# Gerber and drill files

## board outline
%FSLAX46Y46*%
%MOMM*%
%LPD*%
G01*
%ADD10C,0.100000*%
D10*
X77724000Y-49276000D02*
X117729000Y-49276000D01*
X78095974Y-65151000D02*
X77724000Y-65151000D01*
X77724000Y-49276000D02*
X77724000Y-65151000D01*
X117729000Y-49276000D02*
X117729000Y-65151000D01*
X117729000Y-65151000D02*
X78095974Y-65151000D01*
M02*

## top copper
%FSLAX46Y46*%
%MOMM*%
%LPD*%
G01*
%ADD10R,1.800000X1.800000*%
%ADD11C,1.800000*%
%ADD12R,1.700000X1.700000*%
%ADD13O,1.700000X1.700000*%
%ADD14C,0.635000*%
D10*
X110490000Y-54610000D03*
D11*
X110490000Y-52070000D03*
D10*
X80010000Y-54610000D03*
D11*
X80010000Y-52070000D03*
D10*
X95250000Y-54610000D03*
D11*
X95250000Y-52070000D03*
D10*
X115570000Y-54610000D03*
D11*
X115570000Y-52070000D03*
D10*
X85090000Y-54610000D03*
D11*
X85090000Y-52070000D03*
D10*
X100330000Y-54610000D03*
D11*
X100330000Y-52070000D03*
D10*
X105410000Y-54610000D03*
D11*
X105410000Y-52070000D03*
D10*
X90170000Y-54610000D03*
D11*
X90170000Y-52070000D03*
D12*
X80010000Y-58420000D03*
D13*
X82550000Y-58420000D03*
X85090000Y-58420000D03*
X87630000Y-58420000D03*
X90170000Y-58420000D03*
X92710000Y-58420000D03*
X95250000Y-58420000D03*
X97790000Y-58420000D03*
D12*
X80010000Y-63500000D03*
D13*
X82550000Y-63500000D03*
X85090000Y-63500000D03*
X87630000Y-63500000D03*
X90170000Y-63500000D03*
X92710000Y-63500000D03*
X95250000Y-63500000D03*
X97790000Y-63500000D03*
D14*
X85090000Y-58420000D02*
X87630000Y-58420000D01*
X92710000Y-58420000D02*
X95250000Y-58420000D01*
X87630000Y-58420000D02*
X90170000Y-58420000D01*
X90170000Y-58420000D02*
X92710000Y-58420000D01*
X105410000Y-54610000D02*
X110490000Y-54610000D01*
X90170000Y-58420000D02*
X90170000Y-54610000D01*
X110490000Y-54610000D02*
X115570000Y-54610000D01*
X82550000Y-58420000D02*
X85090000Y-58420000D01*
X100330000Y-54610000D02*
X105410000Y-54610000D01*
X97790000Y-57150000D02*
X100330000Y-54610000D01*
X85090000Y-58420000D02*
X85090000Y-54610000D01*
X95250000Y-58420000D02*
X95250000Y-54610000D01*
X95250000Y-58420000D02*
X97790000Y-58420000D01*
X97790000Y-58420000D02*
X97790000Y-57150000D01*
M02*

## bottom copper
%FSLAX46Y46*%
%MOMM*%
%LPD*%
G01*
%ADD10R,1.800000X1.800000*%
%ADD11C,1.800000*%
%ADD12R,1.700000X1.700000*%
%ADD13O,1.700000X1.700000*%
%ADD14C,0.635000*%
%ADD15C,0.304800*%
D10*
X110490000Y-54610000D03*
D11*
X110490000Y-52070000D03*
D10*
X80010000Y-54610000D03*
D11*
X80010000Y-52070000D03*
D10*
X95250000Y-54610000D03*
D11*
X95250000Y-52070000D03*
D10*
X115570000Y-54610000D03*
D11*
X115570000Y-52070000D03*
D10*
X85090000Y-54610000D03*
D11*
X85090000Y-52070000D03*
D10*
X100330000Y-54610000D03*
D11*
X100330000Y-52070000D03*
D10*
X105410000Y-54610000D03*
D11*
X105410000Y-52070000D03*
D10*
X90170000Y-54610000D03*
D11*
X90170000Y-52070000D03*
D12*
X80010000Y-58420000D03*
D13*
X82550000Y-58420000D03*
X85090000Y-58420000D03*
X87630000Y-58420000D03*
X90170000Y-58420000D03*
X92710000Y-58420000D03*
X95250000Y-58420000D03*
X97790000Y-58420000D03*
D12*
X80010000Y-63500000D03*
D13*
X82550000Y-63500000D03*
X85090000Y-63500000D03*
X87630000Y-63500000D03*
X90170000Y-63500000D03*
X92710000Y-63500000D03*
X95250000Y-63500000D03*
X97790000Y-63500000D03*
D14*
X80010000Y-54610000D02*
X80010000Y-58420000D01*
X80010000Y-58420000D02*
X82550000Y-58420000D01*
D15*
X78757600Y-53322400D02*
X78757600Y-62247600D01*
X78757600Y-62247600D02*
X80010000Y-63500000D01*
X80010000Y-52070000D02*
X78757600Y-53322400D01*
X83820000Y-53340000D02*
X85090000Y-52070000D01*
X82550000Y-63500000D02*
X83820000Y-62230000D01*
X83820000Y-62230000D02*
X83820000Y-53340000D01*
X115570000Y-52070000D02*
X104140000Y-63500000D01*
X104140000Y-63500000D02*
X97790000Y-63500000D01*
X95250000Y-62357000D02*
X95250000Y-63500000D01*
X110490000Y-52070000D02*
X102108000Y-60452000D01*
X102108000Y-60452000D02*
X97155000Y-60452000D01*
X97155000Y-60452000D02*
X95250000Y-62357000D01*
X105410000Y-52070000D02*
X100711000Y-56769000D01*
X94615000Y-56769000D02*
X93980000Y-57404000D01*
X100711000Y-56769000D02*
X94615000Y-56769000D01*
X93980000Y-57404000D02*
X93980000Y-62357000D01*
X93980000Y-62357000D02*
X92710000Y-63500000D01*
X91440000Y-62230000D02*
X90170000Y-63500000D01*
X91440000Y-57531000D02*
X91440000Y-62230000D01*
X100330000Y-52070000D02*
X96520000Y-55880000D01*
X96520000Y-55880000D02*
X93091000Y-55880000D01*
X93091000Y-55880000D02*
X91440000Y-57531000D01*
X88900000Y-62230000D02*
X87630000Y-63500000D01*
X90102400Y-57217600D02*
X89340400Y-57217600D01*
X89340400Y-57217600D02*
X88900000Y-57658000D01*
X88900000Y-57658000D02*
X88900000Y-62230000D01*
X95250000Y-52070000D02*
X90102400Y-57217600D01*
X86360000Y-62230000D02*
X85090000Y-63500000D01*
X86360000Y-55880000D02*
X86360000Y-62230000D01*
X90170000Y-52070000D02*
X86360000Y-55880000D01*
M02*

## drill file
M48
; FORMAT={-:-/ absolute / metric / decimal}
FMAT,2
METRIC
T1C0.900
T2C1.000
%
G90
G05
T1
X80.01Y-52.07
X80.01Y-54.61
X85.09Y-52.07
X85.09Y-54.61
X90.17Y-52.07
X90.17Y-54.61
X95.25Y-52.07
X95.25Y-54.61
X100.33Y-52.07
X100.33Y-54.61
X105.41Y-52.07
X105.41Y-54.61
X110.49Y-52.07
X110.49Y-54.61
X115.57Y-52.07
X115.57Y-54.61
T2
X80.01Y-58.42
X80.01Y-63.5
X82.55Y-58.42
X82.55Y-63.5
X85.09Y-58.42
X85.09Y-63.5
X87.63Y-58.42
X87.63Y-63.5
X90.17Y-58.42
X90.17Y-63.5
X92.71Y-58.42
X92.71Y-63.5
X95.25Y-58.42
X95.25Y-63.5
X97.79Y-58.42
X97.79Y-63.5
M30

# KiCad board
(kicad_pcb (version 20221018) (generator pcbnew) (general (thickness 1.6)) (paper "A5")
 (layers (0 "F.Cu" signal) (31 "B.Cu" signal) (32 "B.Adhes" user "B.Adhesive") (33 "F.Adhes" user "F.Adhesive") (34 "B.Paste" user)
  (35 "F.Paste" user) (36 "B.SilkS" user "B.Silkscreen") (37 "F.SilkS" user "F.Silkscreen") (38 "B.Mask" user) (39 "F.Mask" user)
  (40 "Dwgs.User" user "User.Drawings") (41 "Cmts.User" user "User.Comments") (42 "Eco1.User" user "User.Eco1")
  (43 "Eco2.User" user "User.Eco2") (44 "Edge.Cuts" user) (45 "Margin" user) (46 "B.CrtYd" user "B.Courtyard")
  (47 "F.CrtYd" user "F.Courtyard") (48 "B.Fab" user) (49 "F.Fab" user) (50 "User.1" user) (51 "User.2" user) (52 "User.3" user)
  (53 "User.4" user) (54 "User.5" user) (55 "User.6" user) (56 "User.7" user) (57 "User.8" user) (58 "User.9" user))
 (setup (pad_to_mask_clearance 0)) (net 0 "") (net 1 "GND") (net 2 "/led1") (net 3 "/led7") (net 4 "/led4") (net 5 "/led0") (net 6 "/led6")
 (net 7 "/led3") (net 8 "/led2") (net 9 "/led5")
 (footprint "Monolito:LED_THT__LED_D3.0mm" (layer "F.Cu") (at 110.49 54.61 90)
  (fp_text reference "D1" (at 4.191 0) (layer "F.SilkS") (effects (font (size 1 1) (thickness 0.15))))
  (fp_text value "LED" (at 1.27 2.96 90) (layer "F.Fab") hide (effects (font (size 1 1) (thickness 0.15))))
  (pad "1" thru_hole rect (at 0 0 90) (size 1.8 1.8) (drill 0.9) (layers "*.Cu" "*.Mask") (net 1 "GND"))
  (pad "2" thru_hole circle (at 2.54 0 90) (size 1.8 1.8) (drill 0.9) (layers "*.Cu" "*.Mask") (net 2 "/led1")))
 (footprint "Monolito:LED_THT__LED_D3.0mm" (layer "F.Cu") (at 80.01 54.61 90)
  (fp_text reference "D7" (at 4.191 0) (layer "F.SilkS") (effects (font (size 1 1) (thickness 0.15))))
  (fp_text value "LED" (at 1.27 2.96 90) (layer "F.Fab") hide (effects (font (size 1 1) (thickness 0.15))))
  (pad "1" thru_hole rect (at 0 0 90) (size 1.8 1.8) (drill 0.9) (layers "*.Cu" "*.Mask") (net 1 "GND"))
  (pad "2" thru_hole circle (at 2.54 0 90) (size 1.8 1.8) (drill 0.9) (layers "*.Cu" "*.Mask") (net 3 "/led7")))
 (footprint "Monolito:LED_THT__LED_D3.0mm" (layer "F.Cu") (at 95.25 54.61 90)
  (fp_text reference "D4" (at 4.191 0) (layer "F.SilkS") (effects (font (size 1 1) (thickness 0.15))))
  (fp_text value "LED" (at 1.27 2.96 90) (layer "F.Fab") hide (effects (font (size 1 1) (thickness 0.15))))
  (pad "1" thru_hole rect (at 0 0 90) (size 1.8 1.8) (drill 0.9) (layers "*.Cu" "*.Mask") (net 1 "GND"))
  (pad "2" thru_hole circle (at 2.54 0 90) (size 1.8 1.8) (drill 0.9) (layers "*.Cu" "*.Mask") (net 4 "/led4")))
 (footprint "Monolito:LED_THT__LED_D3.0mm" (layer "F.Cu") (at 115.57 54.61 90)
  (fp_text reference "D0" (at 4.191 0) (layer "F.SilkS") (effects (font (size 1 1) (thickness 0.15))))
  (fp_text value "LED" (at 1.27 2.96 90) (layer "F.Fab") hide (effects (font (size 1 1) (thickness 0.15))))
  (pad "1" thru_hole rect (at 0 0 90) (size 1.8 1.8) (drill 0.9) (layers "*.Cu" "*.Mask") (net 1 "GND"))
  (pad "2" thru_hole circle (at 2.54 0 90) (size 1.8 1.8) (drill 0.9) (layers "*.Cu" "*.Mask") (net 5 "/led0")))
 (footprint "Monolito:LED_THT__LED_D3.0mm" (layer "F.Cu") (at 85.09 54.61 90)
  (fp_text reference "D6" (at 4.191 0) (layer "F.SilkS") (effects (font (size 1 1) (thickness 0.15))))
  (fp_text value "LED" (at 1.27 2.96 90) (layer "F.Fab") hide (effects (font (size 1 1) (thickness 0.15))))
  (pad "1" thru_hole rect (at 0 0 90) (size 1.8 1.8) (drill 0.9) (layers "*.Cu" "*.Mask") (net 1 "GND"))
  (pad "2" thru_hole circle (at 2.54 0 90) (size 1.8 1.8) (drill 0.9) (layers "*.Cu" "*.Mask") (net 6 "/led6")))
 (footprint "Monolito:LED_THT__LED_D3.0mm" (layer "F.Cu") (at 100.33 54.61 90)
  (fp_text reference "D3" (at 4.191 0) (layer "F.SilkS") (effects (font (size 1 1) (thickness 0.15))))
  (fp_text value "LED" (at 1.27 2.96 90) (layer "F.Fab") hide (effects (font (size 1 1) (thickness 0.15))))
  (pad "1" thru_hole rect (at 0 0 90) (size 1.8 1.8) (drill 0.9) (layers "*.Cu" "*.Mask") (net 1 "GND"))
  (pad "2" thru_hole circle (at 2.54 0 90) (size 1.8 1.8) (drill 0.9) (layers "*.Cu" "*.Mask") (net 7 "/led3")))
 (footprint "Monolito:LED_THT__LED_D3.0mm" (layer "F.Cu") (at 105.41 54.61 90)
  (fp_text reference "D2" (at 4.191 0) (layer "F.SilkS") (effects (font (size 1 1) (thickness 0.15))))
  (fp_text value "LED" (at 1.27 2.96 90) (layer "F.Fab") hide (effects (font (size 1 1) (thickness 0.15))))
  (pad "1" thru_hole rect (at 0 0 90) (size 1.8 1.8) (drill 0.9) (layers "*.Cu" "*.Mask") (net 1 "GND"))
  (pad "2" thru_hole circle (at 2.54 0 90) (size 1.8 1.8) (drill 0.9) (layers "*.Cu" "*.Mask") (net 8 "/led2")))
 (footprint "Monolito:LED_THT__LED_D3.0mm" (layer "F.Cu") (at 90.17 54.61 90)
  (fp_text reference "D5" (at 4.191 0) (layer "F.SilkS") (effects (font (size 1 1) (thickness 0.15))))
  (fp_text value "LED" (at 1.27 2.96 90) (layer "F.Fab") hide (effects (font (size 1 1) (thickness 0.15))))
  (pad "1" thru_hole rect (at 0 0 90) (size 1.8 1.8) (drill 0.9) (layers "*.Cu" "*.Mask") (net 1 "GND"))
  (pad "2" thru_hole circle (at 2.54 0 90) (size 1.8 1.8) (drill 0.9) (layers "*.Cu" "*.Mask") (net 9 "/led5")))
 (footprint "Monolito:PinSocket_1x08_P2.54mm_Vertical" (layer "B.Cu") (at 80.01 58.42 -90)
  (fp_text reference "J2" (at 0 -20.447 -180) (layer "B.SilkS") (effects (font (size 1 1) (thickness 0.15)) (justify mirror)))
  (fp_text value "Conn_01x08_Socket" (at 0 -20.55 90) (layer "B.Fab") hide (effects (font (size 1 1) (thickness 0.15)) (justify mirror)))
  (pad "1" thru_hole rect (at 0 0 270) (size 1.7 1.7) (drill 1) (layers "*.Cu" "*.Mask") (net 1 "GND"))
  (pad "2" thru_hole oval (at 0 -2.54 270) (size 1.7 1.7) (drill 1) (layers "*.Cu" "*.Mask") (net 1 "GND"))
  (pad "3" thru_hole oval (at 0 -5.08 270) (size 1.7 1.7) (drill 1) (layers "*.Cu" "*.Mask") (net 1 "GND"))
  (pad "4" thru_hole oval (at 0 -7.62 270) (size 1.7 1.7) (drill 1) (layers "*.Cu" "*.Mask") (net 1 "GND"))
  (pad "5" thru_hole oval (at 0 -10.16 270) (size 1.7 1.7) (drill 1) (layers "*.Cu" "*.Mask") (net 1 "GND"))
  (pad "6" thru_hole oval (at 0 -12.7 270) (size 1.7 1.7) (drill 1) (layers "*.Cu" "*.Mask") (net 1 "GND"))
  (pad "7" thru_hole oval (at 0 -15.24 270) (size 1.7 1.7) (drill 1) (layers "*.Cu" "*.Mask") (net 1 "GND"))
  (pad "8" thru_hole oval (at 0 -17.78 270) (size 1.7 1.7) (drill 1) (layers "*.Cu" "*.Mask") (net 1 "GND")))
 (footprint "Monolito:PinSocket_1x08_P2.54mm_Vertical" (layer "B.Cu") (at 80.01 63.5 -90)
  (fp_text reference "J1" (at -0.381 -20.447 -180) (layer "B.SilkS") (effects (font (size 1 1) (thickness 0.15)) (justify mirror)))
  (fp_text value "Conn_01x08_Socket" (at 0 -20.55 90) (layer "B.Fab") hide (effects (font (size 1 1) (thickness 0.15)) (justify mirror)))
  (pad "1" thru_hole rect (at 0 0 270) (size 1.7 1.7) (drill 1) (layers "*.Cu" "*.Mask") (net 3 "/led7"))
  (pad "2" thru_hole oval (at 0 -2.54 270) (size 1.7 1.7) (drill 1) (layers "*.Cu" "*.Mask") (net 6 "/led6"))
  (pad "3" thru_hole oval (at 0 -5.08 270) (size 1.7 1.7) (drill 1) (layers "*.Cu" "*.Mask") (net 9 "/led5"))
  (pad "4" thru_hole oval (at 0 -7.62 270) (size 1.7 1.7) (drill 1) (layers "*.Cu" "*.Mask") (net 4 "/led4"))
  (pad "5" thru_hole oval (at 0 -10.16 270) (size 1.7 1.7) (drill 1) (layers "*.Cu" "*.Mask") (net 7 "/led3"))
  (pad "6" thru_hole oval (at 0 -12.7 270) (size 1.7 1.7) (drill 1) (layers "*.Cu" "*.Mask") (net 8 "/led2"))
  (pad "7" thru_hole oval (at 0 -15.24 270) (size 1.7 1.7) (drill 1) (layers "*.Cu" "*.Mask") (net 2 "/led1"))
  (pad "8" thru_hole oval (at 0 -17.78 270) (size 1.7 1.7) (drill 1) (layers "*.Cu" "*.Mask") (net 5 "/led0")))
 (gr_line (start 77.724 49.276) (end 117.729 49.276) (stroke (width 0.1) (type default)) (layer "Edge.Cuts"))
 (gr_line (start 78.095974 65.151) (end 77.724 65.151) (stroke (width 0.1) (type default)) (layer "Edge.Cuts"))
 (gr_line (start 77.724 49.276) (end 77.724 65.151) (stroke (width 0.1) (type default)) (layer "Edge.Cuts"))
 (gr_line (start 117.729 49.276) (end 117.729 65.151) (stroke (width 0.1) (type default)) (layer "Edge.Cuts"))
 (gr_line (start 117.729 65.151) (end 78.095974 65.151) (stroke (width 0.1) (type default)) (layer "Edge.Cuts"))
 (segment (start 85.09 58.42) (end 87.63 58.42) (width 0.635) (layer "F.Cu") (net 1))
 (segment (start 92.71 58.42) (end 95.25 58.42) (width 0.635) (layer "F.Cu") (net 1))
 (segment (start 87.63 58.42) (end 90.17 58.42) (width 0.635) (layer "F.Cu") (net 1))
 (segment (start 90.17 58.42) (end 92.71 58.42) (width 0.635) (layer "F.Cu") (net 1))
 (segment (start 105.41 54.61) (end 110.49 54.61) (width 0.635) (layer "F.Cu") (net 1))
 (segment (start 90.17 58.42) (end 90.17 54.61) (width 0.635) (layer "F.Cu") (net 1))
 (segment (start 110.49 54.61) (end 115.57 54.61) (width 0.635) (layer "F.Cu") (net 1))
 (segment (start 82.55 58.42) (end 85.09 58.42) (width 0.635) (layer "F.Cu") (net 1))
 (segment (start 100.33 54.61) (end 105.41 54.61) (width 0.635) (layer "F.Cu") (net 1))
 (segment (start 97.79 57.15) (end 100.33 54.61) (width 0.635) (layer "F.Cu") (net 1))
 (segment (start 85.09 58.42) (end 85.09 54.61) (width 0.635) (layer "F.Cu") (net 1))
 (segment (start 95.25 58.42) (end 95.25 54.61) (width 0.635) (layer "F.Cu") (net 1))
 (segment (start 95.25 58.42) (end 97.79 58.42) (width 0.635) (layer "F.Cu") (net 1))
 (segment (start 97.79 58.42) (end 97.79 57.15) (width 0.635) (layer "F.Cu") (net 1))
 (segment (start 80.01 54.61) (end 80.01 58.42) (width 0.635) (layer "B.Cu") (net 1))
 (segment (start 80.01 58.42) (end 82.55 58.42) (width 0.635) (layer "B.Cu") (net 1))
 (segment (start 78.7576 53.3224) (end 78.7576 62.2476) (width 0.3048) (layer "B.Cu") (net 3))
 (segment (start 78.7576 62.2476) (end 80.01 63.5) (width 0.3048) (layer "B.Cu") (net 3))
 (segment (start 80.01 52.07) (end 78.7576 53.3224) (width 0.3048) (layer "B.Cu") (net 3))
 (segment (start 83.82 53.34) (end 85.09 52.07) (width 0.3048) (layer "B.Cu") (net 6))
 (segment (start 82.55 63.5) (end 83.82 62.23) (width 0.3048) (layer "B.Cu") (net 6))
 (segment (start 83.82 62.23) (end 83.82 53.34) (width 0.3048) (layer "B.Cu") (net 6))
 (segment (start 115.57 52.07) (end 104.14 63.5) (width 0.3048) (layer "B.Cu") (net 5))
 (segment (start 104.14 63.5) (end 97.79 63.5) (width 0.3048) (layer "B.Cu") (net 5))
 (segment (start 95.25 62.357) (end 95.25 63.5) (width 0.3048) (layer "B.Cu") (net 2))
 (segment (start 110.49 52.07) (end 102.108 60.452) (width 0.3048) (layer "B.Cu") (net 2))
 (segment (start 102.108 60.452) (end 97.155 60.452) (width 0.3048) (layer "B.Cu") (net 2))
 (segment (start 97.155 60.452) (end 95.25 62.357) (width 0.3048) (layer "B.Cu") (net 2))
 (segment (start 105.41 52.07) (end 100.711 56.769) (width 0.3048) (layer "B.Cu") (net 8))
 (segment (start 94.615 56.769) (end 93.98 57.404) (width 0.3048) (layer "B.Cu") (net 8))
 (segment (start 100.711 56.769) (end 94.615 56.769) (width 0.3048) (layer "B.Cu") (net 8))
 (segment (start 93.98 57.404) (end 93.98 62.357) (width 0.3048) (layer "B.Cu") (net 8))
 (segment (start 93.98 62.357) (end 92.71 63.5) (width 0.3048) (layer "B.Cu") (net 8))
 (segment (start 91.44 62.23) (end 90.17 63.5) (width 0.3048) (layer "B.Cu") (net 7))
 (segment (start 91.44 57.531) (end 91.44 62.23) (width 0.3048) (layer "B.Cu") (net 7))
 (segment (start 100.33 52.07) (end 96.52 55.88) (width 0.3048) (layer "B.Cu") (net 7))
 (segment (start 96.52 55.88) (end 93.091 55.88) (width 0.3048) (layer "B.Cu") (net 7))
 (segment (start 93.091 55.88) (end 91.44 57.531) (width 0.3048) (layer "B.Cu") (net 7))
 (segment (start 88.9 62.23) (end 87.63 63.5) (width 0.3048) (layer "B.Cu") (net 4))
 (segment (start 90.1024 57.2176) (end 89.3404 57.2176) (width 0.3048) (layer "B.Cu") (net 4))
 (segment (start 89.3404 57.2176) (end 88.9 57.658) (width 0.3048) (layer "B.Cu") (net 4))
 (segment (start 88.9 57.658) (end 88.9 62.23) (width 0.3048) (layer "B.Cu") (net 4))
 (segment (start 95.25 52.07) (end 90.1024 57.2176) (width 0.3048) (layer "B.Cu") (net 4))
 (segment (start 86.36 62.23) (end 85.09 63.5) (width 0.3048) (layer "B.Cu") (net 9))
 (segment (start 86.36 55.88) (end 86.36 62.23) (width 0.3048) (layer "B.Cu") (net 9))
 (segment (start 90.17 52.07) (end 86.36 55.88) (width 0.3048) (layer "B.Cu") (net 9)))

